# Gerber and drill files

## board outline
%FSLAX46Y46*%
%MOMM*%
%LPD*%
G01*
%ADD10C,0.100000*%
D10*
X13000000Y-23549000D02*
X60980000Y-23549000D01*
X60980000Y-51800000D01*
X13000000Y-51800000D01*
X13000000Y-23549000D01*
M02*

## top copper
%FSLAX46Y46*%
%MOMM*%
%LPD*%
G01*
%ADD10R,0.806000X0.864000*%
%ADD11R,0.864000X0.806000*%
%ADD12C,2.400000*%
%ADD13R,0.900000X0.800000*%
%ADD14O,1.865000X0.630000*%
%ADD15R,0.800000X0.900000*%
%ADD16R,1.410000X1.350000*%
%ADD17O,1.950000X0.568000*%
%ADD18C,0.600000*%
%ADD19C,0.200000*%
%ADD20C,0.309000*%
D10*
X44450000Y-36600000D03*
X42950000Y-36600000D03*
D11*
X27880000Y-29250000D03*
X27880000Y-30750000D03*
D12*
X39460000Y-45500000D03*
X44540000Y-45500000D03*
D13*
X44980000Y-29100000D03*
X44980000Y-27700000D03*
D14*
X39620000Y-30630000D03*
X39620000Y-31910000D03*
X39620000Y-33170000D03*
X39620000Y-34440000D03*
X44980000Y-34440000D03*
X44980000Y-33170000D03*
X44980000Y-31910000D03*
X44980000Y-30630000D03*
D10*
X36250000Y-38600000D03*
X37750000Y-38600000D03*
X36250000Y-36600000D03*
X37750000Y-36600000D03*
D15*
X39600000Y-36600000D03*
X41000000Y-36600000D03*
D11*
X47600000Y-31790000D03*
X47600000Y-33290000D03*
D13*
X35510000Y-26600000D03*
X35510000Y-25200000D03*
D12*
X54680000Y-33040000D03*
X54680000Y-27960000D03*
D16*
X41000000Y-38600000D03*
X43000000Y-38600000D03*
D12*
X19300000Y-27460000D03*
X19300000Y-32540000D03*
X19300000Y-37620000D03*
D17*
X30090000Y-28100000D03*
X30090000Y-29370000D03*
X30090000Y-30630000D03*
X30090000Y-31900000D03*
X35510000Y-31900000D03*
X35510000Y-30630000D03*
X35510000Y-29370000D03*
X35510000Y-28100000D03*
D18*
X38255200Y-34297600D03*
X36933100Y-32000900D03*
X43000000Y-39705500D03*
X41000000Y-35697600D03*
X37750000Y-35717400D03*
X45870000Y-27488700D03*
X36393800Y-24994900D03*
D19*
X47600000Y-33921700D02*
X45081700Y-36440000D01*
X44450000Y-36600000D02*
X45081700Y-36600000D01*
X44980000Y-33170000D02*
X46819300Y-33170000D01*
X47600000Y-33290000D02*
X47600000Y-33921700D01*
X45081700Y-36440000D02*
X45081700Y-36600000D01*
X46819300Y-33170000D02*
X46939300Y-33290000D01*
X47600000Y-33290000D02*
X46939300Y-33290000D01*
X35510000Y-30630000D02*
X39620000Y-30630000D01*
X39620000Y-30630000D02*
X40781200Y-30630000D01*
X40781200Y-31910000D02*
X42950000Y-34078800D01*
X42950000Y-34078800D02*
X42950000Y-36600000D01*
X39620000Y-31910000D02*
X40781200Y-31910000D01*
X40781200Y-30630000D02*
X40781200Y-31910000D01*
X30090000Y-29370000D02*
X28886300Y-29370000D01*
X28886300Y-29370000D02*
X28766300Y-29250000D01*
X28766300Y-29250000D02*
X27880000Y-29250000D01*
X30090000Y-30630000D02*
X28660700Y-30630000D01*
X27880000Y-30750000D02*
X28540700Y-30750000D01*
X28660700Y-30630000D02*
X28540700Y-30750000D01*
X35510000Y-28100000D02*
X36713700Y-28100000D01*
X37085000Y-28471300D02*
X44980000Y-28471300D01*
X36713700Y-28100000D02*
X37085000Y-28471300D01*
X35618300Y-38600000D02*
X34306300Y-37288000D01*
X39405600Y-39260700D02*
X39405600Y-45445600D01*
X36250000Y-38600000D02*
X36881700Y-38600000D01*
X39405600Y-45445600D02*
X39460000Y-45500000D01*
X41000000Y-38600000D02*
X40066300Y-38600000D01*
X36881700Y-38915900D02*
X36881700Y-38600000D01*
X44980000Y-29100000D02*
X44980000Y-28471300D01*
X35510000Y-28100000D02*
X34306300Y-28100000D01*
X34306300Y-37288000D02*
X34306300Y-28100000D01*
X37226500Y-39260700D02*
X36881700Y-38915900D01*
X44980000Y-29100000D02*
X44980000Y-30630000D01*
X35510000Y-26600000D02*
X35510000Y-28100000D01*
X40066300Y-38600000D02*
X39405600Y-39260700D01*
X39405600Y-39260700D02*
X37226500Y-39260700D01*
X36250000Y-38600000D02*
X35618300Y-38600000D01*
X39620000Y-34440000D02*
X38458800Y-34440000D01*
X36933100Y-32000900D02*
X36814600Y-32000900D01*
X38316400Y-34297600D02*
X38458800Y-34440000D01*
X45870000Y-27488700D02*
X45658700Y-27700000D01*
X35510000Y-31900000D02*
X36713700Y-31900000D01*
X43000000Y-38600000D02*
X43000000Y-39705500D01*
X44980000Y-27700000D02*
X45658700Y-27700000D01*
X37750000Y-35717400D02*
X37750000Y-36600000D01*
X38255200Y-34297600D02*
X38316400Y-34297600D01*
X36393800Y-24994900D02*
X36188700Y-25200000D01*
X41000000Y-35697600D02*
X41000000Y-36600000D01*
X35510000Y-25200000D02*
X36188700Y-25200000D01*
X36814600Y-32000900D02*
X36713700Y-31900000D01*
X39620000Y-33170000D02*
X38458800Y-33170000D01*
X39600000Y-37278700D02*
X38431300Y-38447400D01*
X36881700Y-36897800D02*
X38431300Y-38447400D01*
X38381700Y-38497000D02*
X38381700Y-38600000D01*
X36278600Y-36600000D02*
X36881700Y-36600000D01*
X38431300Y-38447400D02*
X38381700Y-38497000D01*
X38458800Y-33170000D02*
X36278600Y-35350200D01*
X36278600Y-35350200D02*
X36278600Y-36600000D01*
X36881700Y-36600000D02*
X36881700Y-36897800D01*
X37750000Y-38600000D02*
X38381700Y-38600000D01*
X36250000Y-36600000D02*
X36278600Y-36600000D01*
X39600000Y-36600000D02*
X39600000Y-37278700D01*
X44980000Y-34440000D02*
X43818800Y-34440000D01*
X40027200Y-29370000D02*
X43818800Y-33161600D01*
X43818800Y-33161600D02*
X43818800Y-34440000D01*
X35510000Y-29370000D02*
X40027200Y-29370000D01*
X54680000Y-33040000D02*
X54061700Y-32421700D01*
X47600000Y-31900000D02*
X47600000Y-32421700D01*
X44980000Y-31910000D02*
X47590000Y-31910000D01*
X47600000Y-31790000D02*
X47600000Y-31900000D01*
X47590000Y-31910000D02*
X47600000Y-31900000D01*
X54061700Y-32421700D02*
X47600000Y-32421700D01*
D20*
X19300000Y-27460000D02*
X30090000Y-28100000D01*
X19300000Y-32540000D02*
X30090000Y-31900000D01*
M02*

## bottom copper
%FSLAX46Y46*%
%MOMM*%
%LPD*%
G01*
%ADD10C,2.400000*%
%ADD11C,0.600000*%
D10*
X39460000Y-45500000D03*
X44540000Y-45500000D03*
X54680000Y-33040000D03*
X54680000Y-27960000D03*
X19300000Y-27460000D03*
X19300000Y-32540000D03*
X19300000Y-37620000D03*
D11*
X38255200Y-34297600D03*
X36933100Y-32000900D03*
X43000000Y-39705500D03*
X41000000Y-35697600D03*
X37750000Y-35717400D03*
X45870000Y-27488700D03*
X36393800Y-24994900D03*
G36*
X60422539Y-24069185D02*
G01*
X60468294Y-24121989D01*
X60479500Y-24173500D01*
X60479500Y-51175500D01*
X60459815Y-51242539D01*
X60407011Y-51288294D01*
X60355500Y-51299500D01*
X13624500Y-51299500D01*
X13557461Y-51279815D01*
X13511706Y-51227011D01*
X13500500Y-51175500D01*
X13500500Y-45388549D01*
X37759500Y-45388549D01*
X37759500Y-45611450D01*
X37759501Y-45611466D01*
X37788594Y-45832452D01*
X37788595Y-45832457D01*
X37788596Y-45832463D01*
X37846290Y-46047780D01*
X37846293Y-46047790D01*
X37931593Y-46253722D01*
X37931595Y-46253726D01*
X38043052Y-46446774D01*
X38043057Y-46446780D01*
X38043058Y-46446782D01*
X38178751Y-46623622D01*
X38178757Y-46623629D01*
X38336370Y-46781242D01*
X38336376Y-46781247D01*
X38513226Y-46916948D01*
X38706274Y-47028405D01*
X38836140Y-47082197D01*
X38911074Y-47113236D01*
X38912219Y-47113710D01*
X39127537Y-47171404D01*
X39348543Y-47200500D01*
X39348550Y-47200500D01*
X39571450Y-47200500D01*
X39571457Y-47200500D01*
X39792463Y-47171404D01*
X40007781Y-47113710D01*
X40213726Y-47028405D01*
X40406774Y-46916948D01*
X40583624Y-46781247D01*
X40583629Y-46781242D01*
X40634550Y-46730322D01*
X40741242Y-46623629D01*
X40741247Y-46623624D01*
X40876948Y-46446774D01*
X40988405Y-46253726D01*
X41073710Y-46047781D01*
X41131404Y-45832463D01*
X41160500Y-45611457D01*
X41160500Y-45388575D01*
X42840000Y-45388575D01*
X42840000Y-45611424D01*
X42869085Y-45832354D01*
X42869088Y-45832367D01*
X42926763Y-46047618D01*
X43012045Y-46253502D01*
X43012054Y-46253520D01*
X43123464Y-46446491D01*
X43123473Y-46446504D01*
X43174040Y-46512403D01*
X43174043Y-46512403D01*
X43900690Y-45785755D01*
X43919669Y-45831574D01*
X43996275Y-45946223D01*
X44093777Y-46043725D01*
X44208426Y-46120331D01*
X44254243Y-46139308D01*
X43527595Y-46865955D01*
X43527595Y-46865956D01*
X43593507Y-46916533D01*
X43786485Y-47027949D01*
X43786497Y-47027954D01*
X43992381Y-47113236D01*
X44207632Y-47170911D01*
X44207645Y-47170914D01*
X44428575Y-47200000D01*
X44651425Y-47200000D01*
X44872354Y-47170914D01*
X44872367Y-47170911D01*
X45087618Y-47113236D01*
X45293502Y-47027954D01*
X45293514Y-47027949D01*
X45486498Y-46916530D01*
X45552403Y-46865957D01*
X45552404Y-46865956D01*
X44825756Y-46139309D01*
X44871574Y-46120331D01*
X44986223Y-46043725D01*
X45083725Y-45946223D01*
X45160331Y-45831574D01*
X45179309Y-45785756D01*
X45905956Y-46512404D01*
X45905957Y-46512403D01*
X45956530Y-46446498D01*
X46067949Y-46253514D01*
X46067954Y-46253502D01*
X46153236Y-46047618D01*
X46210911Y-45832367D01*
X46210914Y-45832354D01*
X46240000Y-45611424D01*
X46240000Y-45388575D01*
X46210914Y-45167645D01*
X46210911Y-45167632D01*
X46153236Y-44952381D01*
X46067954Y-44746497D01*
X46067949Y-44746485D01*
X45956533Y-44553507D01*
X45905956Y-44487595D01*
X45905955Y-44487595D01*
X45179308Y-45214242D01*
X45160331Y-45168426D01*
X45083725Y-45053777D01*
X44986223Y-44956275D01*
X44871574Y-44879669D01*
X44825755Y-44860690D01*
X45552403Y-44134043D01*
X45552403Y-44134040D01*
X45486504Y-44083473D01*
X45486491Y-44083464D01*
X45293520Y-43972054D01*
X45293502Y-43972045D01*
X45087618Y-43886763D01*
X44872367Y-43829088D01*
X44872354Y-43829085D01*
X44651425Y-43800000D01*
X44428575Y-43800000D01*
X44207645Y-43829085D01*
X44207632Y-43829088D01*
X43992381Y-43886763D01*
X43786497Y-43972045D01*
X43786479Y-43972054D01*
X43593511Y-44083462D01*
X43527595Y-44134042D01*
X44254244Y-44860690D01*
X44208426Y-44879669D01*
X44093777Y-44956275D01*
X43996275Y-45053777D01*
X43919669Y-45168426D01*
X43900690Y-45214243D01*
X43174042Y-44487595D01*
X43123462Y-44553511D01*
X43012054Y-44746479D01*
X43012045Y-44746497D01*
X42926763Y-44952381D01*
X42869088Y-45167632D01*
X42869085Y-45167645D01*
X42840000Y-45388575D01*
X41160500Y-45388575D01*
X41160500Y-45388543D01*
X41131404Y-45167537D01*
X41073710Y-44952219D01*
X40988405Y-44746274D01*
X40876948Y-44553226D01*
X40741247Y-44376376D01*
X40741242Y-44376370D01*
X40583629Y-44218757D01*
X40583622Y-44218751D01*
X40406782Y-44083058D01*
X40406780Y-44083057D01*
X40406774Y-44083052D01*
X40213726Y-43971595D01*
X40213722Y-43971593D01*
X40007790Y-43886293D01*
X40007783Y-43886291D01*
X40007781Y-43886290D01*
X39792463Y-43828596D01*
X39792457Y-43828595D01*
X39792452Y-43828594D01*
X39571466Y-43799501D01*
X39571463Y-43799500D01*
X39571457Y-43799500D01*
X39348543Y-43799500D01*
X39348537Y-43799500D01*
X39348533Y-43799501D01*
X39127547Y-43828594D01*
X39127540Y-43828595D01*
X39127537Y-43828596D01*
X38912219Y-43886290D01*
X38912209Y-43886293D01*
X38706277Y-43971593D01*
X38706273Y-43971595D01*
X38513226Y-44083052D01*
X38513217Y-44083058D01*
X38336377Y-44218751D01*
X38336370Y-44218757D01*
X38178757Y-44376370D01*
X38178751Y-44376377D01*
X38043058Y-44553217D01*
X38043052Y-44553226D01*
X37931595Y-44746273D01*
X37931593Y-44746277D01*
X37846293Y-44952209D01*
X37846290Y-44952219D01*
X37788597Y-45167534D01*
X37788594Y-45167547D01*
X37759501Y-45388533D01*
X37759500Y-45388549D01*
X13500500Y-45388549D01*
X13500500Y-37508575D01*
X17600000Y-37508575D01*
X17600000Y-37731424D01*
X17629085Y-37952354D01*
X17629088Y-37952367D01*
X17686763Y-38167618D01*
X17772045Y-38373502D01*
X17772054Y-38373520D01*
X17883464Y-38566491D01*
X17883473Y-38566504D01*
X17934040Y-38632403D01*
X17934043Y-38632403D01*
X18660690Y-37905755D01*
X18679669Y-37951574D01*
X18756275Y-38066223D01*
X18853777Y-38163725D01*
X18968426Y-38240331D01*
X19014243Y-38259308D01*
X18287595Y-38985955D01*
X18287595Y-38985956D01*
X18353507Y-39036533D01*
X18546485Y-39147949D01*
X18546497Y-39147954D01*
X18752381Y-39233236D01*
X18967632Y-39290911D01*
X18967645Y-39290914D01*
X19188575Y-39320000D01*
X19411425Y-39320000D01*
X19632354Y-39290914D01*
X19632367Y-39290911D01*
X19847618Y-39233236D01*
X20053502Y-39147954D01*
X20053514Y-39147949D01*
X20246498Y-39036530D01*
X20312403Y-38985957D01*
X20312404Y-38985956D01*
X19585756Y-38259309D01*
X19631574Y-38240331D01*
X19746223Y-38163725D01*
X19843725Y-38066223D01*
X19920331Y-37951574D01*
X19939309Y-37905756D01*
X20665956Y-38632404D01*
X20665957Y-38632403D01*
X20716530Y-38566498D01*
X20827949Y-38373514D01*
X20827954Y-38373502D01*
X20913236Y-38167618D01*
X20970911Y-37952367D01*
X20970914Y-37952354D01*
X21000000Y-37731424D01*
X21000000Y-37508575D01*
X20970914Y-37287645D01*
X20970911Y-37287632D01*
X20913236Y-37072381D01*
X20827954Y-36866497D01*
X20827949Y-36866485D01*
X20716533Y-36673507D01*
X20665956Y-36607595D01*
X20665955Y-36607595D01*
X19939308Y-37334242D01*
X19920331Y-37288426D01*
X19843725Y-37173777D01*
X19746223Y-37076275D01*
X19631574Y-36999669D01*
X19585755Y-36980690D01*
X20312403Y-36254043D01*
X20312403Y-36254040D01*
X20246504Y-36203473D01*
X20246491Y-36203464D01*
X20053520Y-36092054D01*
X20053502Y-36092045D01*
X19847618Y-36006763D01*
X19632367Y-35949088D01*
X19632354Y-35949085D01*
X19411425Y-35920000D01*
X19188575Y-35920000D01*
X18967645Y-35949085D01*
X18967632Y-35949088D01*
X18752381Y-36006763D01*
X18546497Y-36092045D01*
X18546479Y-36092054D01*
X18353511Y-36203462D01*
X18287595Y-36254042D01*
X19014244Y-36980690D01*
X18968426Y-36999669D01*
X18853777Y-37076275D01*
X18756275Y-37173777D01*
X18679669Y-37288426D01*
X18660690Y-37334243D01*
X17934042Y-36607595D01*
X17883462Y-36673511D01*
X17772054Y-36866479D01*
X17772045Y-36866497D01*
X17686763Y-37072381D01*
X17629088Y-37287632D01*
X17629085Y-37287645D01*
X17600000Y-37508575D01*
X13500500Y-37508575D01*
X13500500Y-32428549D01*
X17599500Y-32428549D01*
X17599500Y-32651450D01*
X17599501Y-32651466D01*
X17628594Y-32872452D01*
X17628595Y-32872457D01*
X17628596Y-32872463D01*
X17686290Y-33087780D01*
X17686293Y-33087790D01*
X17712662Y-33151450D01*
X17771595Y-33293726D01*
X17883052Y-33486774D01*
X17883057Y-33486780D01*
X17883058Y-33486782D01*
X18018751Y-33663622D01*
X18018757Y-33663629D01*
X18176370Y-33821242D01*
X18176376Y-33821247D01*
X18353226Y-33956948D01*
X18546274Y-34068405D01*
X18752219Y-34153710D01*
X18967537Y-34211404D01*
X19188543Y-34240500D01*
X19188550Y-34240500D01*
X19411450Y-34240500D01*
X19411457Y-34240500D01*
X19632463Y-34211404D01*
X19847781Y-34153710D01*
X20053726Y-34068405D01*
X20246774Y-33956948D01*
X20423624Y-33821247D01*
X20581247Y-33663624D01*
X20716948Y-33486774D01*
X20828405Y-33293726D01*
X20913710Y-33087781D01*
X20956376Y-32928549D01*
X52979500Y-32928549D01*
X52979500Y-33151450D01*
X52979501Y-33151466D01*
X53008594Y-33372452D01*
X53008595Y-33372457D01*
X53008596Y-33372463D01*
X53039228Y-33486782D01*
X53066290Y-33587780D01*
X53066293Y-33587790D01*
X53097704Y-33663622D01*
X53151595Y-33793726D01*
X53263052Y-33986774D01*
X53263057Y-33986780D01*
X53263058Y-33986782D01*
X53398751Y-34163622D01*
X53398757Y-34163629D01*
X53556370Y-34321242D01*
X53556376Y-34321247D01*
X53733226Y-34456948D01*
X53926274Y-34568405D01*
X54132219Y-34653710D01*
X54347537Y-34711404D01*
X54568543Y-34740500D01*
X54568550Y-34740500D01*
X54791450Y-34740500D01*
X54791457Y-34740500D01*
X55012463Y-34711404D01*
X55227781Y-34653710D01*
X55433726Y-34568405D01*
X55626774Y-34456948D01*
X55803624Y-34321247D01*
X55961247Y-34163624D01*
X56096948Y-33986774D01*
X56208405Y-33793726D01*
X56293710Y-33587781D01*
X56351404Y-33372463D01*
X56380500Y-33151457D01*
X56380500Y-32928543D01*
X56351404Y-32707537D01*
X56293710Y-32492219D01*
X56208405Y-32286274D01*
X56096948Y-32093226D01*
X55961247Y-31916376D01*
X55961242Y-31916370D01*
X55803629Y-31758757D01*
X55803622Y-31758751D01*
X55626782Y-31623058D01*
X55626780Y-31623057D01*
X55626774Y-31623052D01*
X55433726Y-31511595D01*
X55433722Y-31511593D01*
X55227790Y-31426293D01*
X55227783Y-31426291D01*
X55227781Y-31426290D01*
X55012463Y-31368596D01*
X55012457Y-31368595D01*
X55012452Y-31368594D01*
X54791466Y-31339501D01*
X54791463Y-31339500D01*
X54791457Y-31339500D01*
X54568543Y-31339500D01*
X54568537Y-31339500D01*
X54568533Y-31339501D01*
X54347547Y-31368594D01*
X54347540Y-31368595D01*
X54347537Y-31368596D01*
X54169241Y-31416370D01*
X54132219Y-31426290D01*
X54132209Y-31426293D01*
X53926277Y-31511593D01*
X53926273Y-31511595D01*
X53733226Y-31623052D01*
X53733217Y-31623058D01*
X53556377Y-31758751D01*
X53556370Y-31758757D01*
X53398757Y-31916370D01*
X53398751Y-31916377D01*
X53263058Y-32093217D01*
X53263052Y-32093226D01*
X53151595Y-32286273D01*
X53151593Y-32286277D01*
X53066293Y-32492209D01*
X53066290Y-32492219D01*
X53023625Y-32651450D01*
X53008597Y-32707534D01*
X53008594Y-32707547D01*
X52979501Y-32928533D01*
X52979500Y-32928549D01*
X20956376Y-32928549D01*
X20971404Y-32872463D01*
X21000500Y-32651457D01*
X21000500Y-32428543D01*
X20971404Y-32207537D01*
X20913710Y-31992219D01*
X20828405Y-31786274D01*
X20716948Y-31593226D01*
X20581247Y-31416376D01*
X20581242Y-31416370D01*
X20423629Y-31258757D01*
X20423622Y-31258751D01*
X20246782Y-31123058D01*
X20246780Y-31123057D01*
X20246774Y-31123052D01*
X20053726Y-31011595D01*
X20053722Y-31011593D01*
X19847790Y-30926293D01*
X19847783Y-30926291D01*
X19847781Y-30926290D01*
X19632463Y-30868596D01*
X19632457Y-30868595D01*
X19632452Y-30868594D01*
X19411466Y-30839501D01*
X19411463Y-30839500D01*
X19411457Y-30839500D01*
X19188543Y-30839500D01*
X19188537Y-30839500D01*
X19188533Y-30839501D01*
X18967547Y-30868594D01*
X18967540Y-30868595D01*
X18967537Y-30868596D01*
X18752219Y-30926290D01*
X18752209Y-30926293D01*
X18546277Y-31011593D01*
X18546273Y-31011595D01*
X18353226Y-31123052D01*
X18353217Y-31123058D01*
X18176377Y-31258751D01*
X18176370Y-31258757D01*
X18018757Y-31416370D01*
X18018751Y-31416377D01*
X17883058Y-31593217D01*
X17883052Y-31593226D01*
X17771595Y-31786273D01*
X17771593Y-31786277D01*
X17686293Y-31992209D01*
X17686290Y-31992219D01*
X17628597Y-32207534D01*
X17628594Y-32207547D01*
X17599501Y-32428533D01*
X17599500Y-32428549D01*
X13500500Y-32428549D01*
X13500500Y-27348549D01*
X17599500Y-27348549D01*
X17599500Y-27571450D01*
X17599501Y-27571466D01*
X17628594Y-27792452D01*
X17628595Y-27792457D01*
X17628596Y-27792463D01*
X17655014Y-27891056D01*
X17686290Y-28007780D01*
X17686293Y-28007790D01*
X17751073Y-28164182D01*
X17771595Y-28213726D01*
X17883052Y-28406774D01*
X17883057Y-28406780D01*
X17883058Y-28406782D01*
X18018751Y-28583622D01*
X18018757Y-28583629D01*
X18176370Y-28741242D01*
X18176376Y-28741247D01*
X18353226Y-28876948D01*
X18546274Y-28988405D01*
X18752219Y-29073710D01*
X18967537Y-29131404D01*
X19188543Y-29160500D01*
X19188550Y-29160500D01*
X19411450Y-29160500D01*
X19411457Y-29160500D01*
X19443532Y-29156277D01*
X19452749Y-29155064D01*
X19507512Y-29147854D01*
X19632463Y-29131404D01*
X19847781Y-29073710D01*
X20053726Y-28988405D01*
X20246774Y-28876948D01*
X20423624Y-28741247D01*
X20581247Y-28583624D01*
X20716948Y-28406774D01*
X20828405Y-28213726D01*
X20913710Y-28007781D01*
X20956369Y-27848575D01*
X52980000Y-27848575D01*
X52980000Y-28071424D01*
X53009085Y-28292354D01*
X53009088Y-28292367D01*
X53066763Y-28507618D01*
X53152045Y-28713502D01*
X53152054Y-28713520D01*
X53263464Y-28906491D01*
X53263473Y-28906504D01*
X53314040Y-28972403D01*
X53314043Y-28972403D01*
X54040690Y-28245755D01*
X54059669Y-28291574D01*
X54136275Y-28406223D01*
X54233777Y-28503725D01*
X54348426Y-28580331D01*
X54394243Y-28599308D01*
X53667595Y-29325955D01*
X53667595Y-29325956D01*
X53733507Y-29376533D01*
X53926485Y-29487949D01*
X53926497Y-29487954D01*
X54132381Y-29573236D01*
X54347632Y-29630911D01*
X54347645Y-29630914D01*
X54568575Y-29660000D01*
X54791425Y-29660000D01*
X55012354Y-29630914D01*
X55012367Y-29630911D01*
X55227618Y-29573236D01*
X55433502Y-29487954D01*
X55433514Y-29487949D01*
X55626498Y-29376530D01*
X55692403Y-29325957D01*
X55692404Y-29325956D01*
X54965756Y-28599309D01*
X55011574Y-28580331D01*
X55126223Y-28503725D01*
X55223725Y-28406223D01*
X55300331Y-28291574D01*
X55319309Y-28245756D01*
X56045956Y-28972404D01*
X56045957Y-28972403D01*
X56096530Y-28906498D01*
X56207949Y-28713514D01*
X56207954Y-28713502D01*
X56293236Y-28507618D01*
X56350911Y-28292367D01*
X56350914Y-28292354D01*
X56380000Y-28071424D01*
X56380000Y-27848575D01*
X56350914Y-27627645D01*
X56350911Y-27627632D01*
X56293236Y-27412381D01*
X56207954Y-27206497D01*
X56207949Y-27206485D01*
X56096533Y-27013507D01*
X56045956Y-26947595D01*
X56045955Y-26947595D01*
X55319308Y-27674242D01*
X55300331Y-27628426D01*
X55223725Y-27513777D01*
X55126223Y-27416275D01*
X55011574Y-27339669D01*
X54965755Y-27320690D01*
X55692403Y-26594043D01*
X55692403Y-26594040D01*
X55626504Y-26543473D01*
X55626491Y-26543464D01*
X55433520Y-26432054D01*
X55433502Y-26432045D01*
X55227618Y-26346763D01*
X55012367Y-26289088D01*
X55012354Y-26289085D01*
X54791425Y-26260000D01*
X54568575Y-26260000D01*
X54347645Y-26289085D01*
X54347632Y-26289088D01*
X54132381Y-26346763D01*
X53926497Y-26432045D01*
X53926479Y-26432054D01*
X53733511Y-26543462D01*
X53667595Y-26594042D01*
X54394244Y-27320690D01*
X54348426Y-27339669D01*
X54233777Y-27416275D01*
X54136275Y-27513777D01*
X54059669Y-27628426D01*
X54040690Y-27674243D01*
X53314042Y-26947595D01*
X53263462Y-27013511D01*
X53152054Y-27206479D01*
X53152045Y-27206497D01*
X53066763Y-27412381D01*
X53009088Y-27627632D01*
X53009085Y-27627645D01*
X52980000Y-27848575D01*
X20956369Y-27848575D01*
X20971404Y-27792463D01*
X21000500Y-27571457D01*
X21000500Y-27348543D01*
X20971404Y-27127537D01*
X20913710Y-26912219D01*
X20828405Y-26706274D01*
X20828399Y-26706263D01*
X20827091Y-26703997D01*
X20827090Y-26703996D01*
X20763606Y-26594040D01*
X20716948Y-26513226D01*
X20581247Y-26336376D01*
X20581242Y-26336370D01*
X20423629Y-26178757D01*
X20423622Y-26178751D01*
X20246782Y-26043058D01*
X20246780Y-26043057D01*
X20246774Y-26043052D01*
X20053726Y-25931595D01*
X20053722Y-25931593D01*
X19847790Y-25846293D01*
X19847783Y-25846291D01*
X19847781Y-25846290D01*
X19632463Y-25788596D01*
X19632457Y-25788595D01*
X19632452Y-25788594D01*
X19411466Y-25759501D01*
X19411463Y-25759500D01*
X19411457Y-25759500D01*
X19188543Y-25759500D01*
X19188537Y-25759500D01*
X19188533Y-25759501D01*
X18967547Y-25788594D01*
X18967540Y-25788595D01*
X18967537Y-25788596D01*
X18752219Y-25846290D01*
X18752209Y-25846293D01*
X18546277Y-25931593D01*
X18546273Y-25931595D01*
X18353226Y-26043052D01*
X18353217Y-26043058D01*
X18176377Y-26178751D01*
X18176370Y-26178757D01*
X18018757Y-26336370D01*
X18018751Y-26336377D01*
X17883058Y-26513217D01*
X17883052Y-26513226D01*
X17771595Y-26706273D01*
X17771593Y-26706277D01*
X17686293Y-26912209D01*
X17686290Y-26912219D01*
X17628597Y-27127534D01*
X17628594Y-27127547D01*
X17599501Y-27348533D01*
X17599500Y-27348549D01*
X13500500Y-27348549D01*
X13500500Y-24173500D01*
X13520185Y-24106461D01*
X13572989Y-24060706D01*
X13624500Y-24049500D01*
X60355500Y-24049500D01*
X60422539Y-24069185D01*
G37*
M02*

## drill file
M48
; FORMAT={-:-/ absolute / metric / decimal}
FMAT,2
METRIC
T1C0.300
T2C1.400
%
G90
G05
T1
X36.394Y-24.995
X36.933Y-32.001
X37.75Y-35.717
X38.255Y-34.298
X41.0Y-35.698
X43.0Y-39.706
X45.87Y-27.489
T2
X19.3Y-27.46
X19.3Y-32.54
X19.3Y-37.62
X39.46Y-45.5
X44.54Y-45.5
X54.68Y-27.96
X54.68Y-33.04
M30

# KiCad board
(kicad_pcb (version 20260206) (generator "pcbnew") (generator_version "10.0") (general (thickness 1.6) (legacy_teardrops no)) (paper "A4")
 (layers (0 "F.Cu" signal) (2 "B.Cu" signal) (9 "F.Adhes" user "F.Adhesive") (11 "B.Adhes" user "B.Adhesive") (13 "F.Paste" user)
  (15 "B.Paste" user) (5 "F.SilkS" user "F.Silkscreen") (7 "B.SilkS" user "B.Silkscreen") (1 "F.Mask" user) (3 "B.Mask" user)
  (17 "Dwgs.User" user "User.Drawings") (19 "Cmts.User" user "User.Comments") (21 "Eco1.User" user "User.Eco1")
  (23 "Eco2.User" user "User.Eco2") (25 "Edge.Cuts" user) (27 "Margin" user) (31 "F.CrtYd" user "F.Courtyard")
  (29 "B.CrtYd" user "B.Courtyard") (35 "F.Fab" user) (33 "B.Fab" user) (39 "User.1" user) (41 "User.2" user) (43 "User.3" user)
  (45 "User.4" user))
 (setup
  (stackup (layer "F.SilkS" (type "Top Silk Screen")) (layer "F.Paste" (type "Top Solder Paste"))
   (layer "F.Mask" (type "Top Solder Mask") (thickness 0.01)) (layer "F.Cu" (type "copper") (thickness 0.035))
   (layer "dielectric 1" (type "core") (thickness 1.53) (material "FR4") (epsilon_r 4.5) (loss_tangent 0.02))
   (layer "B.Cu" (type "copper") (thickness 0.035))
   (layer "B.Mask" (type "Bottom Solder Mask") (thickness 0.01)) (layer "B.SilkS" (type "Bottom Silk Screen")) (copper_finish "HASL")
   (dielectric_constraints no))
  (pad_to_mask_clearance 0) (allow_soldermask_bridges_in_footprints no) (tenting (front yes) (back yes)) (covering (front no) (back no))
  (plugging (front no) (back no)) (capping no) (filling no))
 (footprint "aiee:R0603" (layer "F.Cu") (at 43.7 36.6 180)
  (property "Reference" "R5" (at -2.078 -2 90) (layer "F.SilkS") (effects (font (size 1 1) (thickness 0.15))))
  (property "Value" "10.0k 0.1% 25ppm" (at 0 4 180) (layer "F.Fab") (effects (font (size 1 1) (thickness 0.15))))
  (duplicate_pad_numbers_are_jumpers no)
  (pad "1" smd rect (at -0.75 0 180) (size 0.806 0.864) (layers "F.Cu" "F.Mask" "F.Paste") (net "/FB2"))
  (pad "2" smd rect (at 0.75 0 180) (size 0.806 0.864) (layers "F.Cu" "F.Mask" "F.Paste") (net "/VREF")))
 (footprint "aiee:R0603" (layer "F.Cu") (at 27.88 30 -90)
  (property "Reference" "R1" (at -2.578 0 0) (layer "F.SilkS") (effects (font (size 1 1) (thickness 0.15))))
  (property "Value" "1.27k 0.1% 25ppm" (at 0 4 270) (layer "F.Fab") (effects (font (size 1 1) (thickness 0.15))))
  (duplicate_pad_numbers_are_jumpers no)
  (pad "1" smd rect (at -0.75 0 270) (size 0.806 0.864) (layers "F.Cu" "F.Mask" "F.Paste") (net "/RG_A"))
  (pad "2" smd rect (at 0.75 0 270) (size 0.806 0.864) (layers "F.Cu" "F.Mask" "F.Paste") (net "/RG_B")))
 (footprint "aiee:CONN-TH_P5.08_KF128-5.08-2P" (layer "F.Cu") (at 42 45.5)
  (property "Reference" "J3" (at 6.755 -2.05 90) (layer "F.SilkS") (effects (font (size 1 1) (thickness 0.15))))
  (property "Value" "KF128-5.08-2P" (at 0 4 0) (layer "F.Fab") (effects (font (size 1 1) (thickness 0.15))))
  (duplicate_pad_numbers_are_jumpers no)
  (pad "1" thru_hole circle (at -2.54 0) (size 2.4 2.4) (drill 1.399998) (layers "*.Cu" "*.Mask") (remove_unused_layers no) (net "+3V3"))
  (pad "2" thru_hole circle (at 2.54 0) (size 2.4 2.4) (drill 1.399998) (layers "*.Cu" "*.Mask") (remove_unused_layers no) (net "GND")))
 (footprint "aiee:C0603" (layer "F.Cu") (at 44.98 28.4 90)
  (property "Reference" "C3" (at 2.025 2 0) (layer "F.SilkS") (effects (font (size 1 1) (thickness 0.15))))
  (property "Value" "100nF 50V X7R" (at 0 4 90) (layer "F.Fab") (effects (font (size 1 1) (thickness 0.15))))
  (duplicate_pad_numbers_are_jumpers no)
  (pad "1" smd rect (at -0.7 0 90) (size 0.8 0.9) (layers "F.Cu" "F.Mask" "F.Paste") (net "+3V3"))
  (pad "2" smd rect (at 0.7 0 90) (size 0.8 0.9) (layers "F.Cu" "F.Mask" "F.Paste") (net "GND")))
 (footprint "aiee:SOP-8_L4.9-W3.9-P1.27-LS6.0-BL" (layer "F.Cu") (at 42.3 32.54 -90)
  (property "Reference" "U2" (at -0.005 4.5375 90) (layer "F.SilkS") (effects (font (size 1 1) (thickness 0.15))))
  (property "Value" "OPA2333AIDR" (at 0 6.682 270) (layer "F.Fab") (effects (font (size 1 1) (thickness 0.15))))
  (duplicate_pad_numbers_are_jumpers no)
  (pad "1" smd oval (at -1.91 2.68 270) (size 0.63 1.865) (layers "F.Cu" "F.Mask" "F.Paste") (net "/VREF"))
  (pad "2" smd oval (at -0.63 2.68 270) (size 0.63 1.865) (layers "F.Cu" "F.Mask" "F.Paste") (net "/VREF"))
  (pad "3" smd oval (at 0.63 2.68 270) (size 0.63 1.865) (layers "F.Cu" "F.Mask" "F.Paste") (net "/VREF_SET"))
  (pad "4" smd oval (at 1.9 2.68 270) (size 0.63 1.865) (layers "F.Cu" "F.Mask" "F.Paste") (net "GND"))
  (pad "5" smd oval (at 1.9 -2.68 270) (size 0.63 1.865) (layers "F.Cu" "F.Mask" "F.Paste") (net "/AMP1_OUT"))
  (pad "6" smd oval (at 0.63 -2.68 270) (size 0.63 1.865) (layers "F.Cu" "F.Mask" "F.Paste") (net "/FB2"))
  (pad "7" smd oval (at -0.63 -2.68 270) (size 0.63 1.865) (layers "F.Cu" "F.Mask" "F.Paste") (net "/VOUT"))
  (pad "8" smd oval (at -1.91 -2.68 270) (size 0.63 1.865) (layers "F.Cu" "F.Mask" "F.Paste") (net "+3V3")))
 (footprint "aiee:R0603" (layer "F.Cu") (at 37 38.6)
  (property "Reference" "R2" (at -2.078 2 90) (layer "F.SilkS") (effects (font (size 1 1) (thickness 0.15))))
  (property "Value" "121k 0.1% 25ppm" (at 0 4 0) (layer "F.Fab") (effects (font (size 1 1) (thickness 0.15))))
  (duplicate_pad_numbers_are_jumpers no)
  (pad "1" smd rect (at -0.75 0) (size 0.806 0.864) (layers "F.Cu" "F.Mask" "F.Paste") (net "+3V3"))
  (pad "2" smd rect (at 0.75 0) (size 0.806 0.864) (layers "F.Cu" "F.Mask" "F.Paste") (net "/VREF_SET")))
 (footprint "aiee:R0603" (layer "F.Cu") (at 37 36.6)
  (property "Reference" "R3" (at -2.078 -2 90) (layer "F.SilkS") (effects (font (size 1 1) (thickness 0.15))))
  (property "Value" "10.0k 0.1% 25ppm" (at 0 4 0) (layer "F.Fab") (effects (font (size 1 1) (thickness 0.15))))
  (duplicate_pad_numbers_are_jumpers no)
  (pad "1" smd rect (at -0.75 0) (size 0.806 0.864) (layers "F.Cu" "F.Mask" "F.Paste") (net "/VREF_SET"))
  (pad "2" smd rect (at 0.75 0) (size 0.806 0.864) (layers "F.Cu" "F.Mask" "F.Paste") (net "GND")))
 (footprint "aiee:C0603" (layer "F.Cu") (at 40.3 36.6)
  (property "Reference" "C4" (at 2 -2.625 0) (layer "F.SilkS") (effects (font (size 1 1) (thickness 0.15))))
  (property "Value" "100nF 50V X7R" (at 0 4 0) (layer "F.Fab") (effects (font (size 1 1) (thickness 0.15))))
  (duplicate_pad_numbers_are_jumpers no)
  (pad "1" smd rect (at -0.7 0) (size 0.8 0.9) (layers "F.Cu" "F.Mask" "F.Paste") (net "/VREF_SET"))
  (pad "2" smd rect (at 0.7 0) (size 0.8 0.9) (layers "F.Cu" "F.Mask" "F.Paste") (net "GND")))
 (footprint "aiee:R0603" (layer "F.Cu") (at 47.6 32.54 -90)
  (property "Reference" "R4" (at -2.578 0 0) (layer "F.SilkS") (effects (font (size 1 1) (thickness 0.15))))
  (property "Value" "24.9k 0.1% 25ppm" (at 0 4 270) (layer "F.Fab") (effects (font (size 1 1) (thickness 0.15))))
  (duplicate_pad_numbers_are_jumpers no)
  (pad "1" smd rect (at -0.75 0 270) (size 0.806 0.864) (layers "F.Cu" "F.Mask" "F.Paste") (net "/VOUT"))
  (pad "2" smd rect (at 0.75 0 270) (size 0.806 0.864) (layers "F.Cu" "F.Mask" "F.Paste") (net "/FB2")))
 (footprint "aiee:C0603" (layer "F.Cu") (at 35.51 25.9 90)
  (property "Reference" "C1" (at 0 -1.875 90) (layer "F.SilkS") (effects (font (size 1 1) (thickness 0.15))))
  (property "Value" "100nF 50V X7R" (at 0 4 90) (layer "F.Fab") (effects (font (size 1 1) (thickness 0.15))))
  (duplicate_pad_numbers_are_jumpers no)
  (pad "1" smd rect (at -0.7 0 90) (size 0.8 0.9) (layers "F.Cu" "F.Mask" "F.Paste") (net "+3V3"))
  (pad "2" smd rect (at 0.7 0 90) (size 0.8 0.9) (layers "F.Cu" "F.Mask" "F.Paste") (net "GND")))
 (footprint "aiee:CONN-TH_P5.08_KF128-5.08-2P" (layer "F.Cu") (at 54.68 30.5 90)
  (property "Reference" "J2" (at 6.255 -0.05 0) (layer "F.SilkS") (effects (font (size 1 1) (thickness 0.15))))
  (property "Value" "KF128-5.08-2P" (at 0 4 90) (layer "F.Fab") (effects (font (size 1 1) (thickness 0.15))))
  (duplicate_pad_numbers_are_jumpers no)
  (pad "1" thru_hole circle (at -2.54 0 90) (size 2.4 2.4) (drill 1.399998) (layers "*.Cu" "*.Mask") (remove_unused_layers no) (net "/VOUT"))
  (pad "2" thru_hole circle (at 2.54 0 90) (size 2.4 2.4) (drill 1.399998) (layers "*.Cu" "*.Mask") (remove_unused_layers no) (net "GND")))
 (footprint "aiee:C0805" (layer "F.Cu") (at 42 38.6)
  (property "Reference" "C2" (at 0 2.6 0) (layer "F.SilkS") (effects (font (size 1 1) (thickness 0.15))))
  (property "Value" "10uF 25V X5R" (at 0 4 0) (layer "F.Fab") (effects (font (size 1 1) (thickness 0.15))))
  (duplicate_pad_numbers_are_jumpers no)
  (pad "1" smd rect (at -1 0) (size 1.41 1.35) (layers "F.Cu" "F.Mask" "F.Paste") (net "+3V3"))
  (pad "2" smd rect (at 1 0) (size 1.41 1.35) (layers "F.Cu" "F.Mask" "F.Paste") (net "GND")))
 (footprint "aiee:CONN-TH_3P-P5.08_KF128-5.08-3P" (layer "F.Cu") (at 19.3 32.54 -90)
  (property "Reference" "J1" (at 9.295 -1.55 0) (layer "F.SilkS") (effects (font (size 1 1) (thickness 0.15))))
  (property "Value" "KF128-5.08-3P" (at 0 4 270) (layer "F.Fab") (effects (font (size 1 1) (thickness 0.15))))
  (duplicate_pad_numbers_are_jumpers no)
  (pad "1" thru_hole circle (at -5.08 0 270) (size 2.4 2.4) (drill 1.399998) (layers "*.Cu" "*.Mask") (remove_unused_layers no)
   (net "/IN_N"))
  (pad "2" thru_hole circle (at 0 0 270) (size 2.4 2.4) (drill 1.399998) (layers "*.Cu" "*.Mask") (remove_unused_layers no) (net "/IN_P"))
  (pad "3" thru_hole circle (at 5.08 0 270) (size 2.4 2.4) (drill 1.399998) (layers "*.Cu" "*.Mask") (remove_unused_layers no) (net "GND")))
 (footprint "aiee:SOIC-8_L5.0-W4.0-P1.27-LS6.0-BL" (layer "F.Cu") (at 32.8 30 -90)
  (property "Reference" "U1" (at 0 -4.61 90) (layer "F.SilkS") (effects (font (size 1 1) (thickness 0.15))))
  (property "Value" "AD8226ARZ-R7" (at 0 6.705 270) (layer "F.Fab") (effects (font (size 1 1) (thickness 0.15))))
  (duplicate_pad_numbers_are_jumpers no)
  (pad "1" smd oval (at -1.9 2.71 270) (size 0.568 1.95) (layers "F.Cu" "F.Mask" "F.Paste") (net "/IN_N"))
  (pad "2" smd oval (at -0.63 2.71 270) (size 0.568 1.95) (layers "F.Cu" "F.Mask" "F.Paste") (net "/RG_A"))
  (pad "3" smd oval (at 0.63 2.71 270) (size 0.568 1.95) (layers "F.Cu" "F.Mask" "F.Paste") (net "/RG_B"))
  (pad "4" smd oval (at 1.9 2.71 270) (size 0.568 1.95) (layers "F.Cu" "F.Mask" "F.Paste") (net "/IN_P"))
  (pad "5" smd oval (at 1.9 -2.71 270) (size 0.568 1.95) (layers "F.Cu" "F.Mask" "F.Paste") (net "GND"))
  (pad "6" smd oval (at 0.63 -2.71 270) (size 0.568 1.95) (layers "F.Cu" "F.Mask" "F.Paste") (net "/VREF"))
  (pad "7" smd oval (at -0.63 -2.71 270) (size 0.568 1.95) (layers "F.Cu" "F.Mask" "F.Paste") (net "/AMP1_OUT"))
  (pad "8" smd oval (at -1.9 -2.71 270) (size 0.568 1.95) (layers "F.Cu" "F.Mask" "F.Paste") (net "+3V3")))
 (gr_rect (start 13 23.549) (end 60.98 51.8) (stroke (width 0.1) (type default)) (fill no) (layer "Edge.Cuts"))
 (segment (start 47.6 33.9217) (end 45.0817 36.44) (width 0.2) (layer "F.Cu") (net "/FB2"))
 (segment (start 44.45 36.6) (end 45.0817 36.6) (width 0.2) (layer "F.Cu") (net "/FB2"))
 (segment (start 44.98 33.17) (end 46.8193 33.17) (width 0.2) (layer "F.Cu") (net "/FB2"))
 (segment (start 47.6 33.29) (end 47.6 33.9217) (width 0.2) (layer "F.Cu") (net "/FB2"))
 (segment (start 45.0817 36.44) (end 45.0817 36.6) (width 0.2) (layer "F.Cu") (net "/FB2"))
 (segment (start 46.8193 33.17) (end 46.9393 33.29) (width 0.2) (layer "F.Cu") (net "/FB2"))
 (segment (start 47.6 33.29) (end 46.9393 33.29) (width 0.2) (layer "F.Cu") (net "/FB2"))
 (segment (start 35.51 30.63) (end 39.62 30.63) (width 0.2) (layer "F.Cu") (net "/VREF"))
 (segment (start 39.62 30.63) (end 40.7812 30.63) (width 0.2) (layer "F.Cu") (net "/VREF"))
 (segment (start 40.7812 31.91) (end 42.95 34.0788) (width 0.2) (layer "F.Cu") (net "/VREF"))
 (segment (start 42.95 34.0788) (end 42.95 36.6) (width 0.2) (layer "F.Cu") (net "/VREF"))
 (segment (start 39.62 31.91) (end 40.7812 31.91) (width 0.2) (layer "F.Cu") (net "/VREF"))
 (segment (start 40.7812 30.63) (end 40.7812 31.91) (width 0.2) (layer "F.Cu") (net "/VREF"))
 (segment (start 30.09 29.37) (end 28.8863 29.37) (width 0.2) (layer "F.Cu") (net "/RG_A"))
 (segment (start 28.8863 29.37) (end 28.7663 29.25) (width 0.2) (layer "F.Cu") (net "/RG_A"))
 (segment (start 28.7663 29.25) (end 27.88 29.25) (width 0.2) (layer "F.Cu") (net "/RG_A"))
 (segment (start 30.09 30.63) (end 28.6607 30.63) (width 0.2) (layer "F.Cu") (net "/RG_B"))
 (segment (start 27.88 30.75) (end 28.5407 30.75) (width 0.2) (layer "F.Cu") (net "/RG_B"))
 (segment (start 28.6607 30.63) (end 28.5407 30.75) (width 0.2) (layer "F.Cu") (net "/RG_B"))
 (segment (start 35.51 28.1) (end 36.7137 28.1) (width 0.2) (layer "F.Cu") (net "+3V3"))
 (segment (start 37.085 28.4713) (end 44.98 28.4713) (width 0.2) (layer "F.Cu") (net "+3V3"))
 (segment (start 36.7137 28.1) (end 37.085 28.4713) (width 0.2) (layer "F.Cu") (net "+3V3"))
 (segment (start 35.6183 38.6) (end 34.3063 37.288) (width 0.2) (layer "F.Cu") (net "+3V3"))
 (segment (start 39.4056 39.2607) (end 39.4056 45.4456) (width 0.2) (layer "F.Cu") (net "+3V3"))
 (segment (start 36.25 38.6) (end 36.8817 38.6) (width 0.2) (layer "F.Cu") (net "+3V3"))
 (segment (start 39.4056 45.4456) (end 39.46 45.5) (width 0.2) (layer "F.Cu") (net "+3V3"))
 (segment (start 41 38.6) (end 40.0663 38.6) (width 0.2) (layer "F.Cu") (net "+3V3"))
 (segment (start 36.8817 38.9159) (end 36.8817 38.6) (width 0.2) (layer "F.Cu") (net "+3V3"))
 (segment (start 44.98 29.1) (end 44.98 28.4713) (width 0.2) (layer "F.Cu") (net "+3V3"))
 (segment (start 35.51 28.1) (end 34.3063 28.1) (width 0.2) (layer "F.Cu") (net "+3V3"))
 (segment (start 34.3063 37.288) (end 34.3063 28.1) (width 0.2) (layer "F.Cu") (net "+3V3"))
 (segment (start 37.2265 39.2607) (end 36.8817 38.9159) (width 0.2) (layer "F.Cu") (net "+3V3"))
 (segment (start 44.98 29.1) (end 44.98 30.63) (width 0.2) (layer "F.Cu") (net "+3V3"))
 (segment (start 35.51 26.6) (end 35.51 28.1) (width 0.2) (layer "F.Cu") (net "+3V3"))
 (segment (start 40.0663 38.6) (end 39.4056 39.2607) (width 0.2) (layer "F.Cu") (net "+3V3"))
 (segment (start 39.4056 39.2607) (end 37.2265 39.2607) (width 0.2) (layer "F.Cu") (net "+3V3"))
 (segment (start 36.25 38.6) (end 35.6183 38.6) (width 0.2) (layer "F.Cu") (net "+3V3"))
 (segment (start 39.62 34.44) (end 38.4588 34.44) (width 0.2) (layer "F.Cu") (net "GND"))
 (segment (start 36.9331 32.0009) (end 36.8146 32.0009) (width 0.2) (layer "F.Cu") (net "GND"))
 (segment (start 38.3164 34.2976) (end 38.4588 34.44) (width 0.2) (layer "F.Cu") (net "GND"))
 (segment (start 45.87 27.4887) (end 45.6587 27.7) (width 0.2) (layer "F.Cu") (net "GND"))
 (segment (start 35.51 31.9) (end 36.7137 31.9) (width 0.2) (layer "F.Cu") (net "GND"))
 (segment (start 43 38.6) (end 43 39.7055) (width 0.2) (layer "F.Cu") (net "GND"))
 (segment (start 44.98 27.7) (end 45.6587 27.7) (width 0.2) (layer "F.Cu") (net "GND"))
 (segment (start 37.75 35.7174) (end 37.75 36.6) (width 0.2) (layer "F.Cu") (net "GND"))
 (segment (start 38.2552 34.2976) (end 38.3164 34.2976) (width 0.2) (layer "F.Cu") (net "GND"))
 (segment (start 36.3938 24.9949) (end 36.1887 25.2) (width 0.2) (layer "F.Cu") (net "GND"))
 (segment (start 41 35.6976) (end 41 36.6) (width 0.2) (layer "F.Cu") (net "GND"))
 (segment (start 35.51 25.2) (end 36.1887 25.2) (width 0.2) (layer "F.Cu") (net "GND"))
 (segment (start 36.8146 32.0009) (end 36.7137 31.9) (width 0.2) (layer "F.Cu") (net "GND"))
 (via (at 38.2552 34.2976) (size 0.6) (drill 0.3) (layers "F.Cu" "B.Cu") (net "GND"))
 (via (at 36.9331 32.0009) (size 0.6) (drill 0.3) (layers "F.Cu" "B.Cu") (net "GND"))
 (via (at 43 39.7055) (size 0.6) (drill 0.3) (layers "F.Cu" "B.Cu") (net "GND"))
 (via (at 41 35.6976) (size 0.6) (drill 0.3) (layers "F.Cu" "B.Cu") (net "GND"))
 (via (at 37.75 35.7174) (size 0.6) (drill 0.3) (layers "F.Cu" "B.Cu") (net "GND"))
 (via (at 45.87 27.4887) (size 0.6) (drill 0.3) (layers "F.Cu" "B.Cu") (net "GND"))
 (via (at 36.3938 24.9949) (size 0.6) (drill 0.3) (layers "F.Cu" "B.Cu") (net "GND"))
 (segment (start 39.62 33.17) (end 38.4588 33.17) (width 0.2) (layer "F.Cu") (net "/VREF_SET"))
 (segment (start 39.6 37.2787) (end 38.4313 38.4474) (width 0.2) (layer "F.Cu") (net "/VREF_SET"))
 (segment (start 36.8817 36.8978) (end 38.4313 38.4474) (width 0.2) (layer "F.Cu") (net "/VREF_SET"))
 (segment (start 38.3817 38.497) (end 38.3817 38.6) (width 0.2) (layer "F.Cu") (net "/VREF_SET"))
 (segment (start 36.2786 36.6) (end 36.8817 36.6) (width 0.2) (layer "F.Cu") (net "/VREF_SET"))
 (segment (start 38.4313 38.4474) (end 38.3817 38.497) (width 0.2) (layer "F.Cu") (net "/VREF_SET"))
 (segment (start 38.4588 33.17) (end 36.2786 35.3502) (width 0.2) (layer "F.Cu") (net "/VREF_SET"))
 (segment (start 36.2786 35.3502) (end 36.2786 36.6) (width 0.2) (layer "F.Cu") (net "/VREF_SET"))
 (segment (start 36.8817 36.6) (end 36.8817 36.8978) (width 0.2) (layer "F.Cu") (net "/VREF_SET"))
 (segment (start 37.75 38.6) (end 38.3817 38.6) (width 0.2) (layer "F.Cu") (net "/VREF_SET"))
 (segment (start 36.25 36.6) (end 36.2786 36.6) (width 0.2) (layer "F.Cu") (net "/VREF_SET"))
 (segment (start 39.6 36.6) (end 39.6 37.2787) (width 0.2) (layer "F.Cu") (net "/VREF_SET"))
 (segment (start 44.98 34.44) (end 43.8188 34.44) (width 0.2) (layer "F.Cu") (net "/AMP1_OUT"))
 (segment (start 40.0272 29.37) (end 43.8188 33.1616) (width 0.2) (layer "F.Cu") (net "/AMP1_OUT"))
 (segment (start 43.8188 33.1616) (end 43.8188 34.44) (width 0.2) (layer "F.Cu") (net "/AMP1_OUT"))
 (segment (start 35.51 29.37) (end 40.0272 29.37) (width 0.2) (layer "F.Cu") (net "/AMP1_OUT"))
 (segment (start 54.68 33.04) (end 54.0617 32.4217) (width 0.2) (layer "F.Cu") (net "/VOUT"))
 (segment (start 47.6 31.9) (end 47.6 32.4217) (width 0.2) (layer "F.Cu") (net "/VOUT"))
 (segment (start 44.98 31.91) (end 47.59 31.91) (width 0.2) (layer "F.Cu") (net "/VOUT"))
 (segment (start 47.6 31.79) (end 47.6 31.9) (width 0.2) (layer "F.Cu") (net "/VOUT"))
 (segment (start 47.59 31.91) (end 47.6 31.9) (width 0.2) (layer "F.Cu") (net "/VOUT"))
 (segment (start 54.0617 32.4217) (end 47.6 32.4217) (width 0.2) (layer "F.Cu") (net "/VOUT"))
 (segment (start 19.3 27.46) (end 30.09 28.1) (width 0.309) (layer "F.Cu") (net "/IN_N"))
 (segment (start 19.3 32.54) (end 30.09 31.9) (width 0.309) (layer "F.Cu") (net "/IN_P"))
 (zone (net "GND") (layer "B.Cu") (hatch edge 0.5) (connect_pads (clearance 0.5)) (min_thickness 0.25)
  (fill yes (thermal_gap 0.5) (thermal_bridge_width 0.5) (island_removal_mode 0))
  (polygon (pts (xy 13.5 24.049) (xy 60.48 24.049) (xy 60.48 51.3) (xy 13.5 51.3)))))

